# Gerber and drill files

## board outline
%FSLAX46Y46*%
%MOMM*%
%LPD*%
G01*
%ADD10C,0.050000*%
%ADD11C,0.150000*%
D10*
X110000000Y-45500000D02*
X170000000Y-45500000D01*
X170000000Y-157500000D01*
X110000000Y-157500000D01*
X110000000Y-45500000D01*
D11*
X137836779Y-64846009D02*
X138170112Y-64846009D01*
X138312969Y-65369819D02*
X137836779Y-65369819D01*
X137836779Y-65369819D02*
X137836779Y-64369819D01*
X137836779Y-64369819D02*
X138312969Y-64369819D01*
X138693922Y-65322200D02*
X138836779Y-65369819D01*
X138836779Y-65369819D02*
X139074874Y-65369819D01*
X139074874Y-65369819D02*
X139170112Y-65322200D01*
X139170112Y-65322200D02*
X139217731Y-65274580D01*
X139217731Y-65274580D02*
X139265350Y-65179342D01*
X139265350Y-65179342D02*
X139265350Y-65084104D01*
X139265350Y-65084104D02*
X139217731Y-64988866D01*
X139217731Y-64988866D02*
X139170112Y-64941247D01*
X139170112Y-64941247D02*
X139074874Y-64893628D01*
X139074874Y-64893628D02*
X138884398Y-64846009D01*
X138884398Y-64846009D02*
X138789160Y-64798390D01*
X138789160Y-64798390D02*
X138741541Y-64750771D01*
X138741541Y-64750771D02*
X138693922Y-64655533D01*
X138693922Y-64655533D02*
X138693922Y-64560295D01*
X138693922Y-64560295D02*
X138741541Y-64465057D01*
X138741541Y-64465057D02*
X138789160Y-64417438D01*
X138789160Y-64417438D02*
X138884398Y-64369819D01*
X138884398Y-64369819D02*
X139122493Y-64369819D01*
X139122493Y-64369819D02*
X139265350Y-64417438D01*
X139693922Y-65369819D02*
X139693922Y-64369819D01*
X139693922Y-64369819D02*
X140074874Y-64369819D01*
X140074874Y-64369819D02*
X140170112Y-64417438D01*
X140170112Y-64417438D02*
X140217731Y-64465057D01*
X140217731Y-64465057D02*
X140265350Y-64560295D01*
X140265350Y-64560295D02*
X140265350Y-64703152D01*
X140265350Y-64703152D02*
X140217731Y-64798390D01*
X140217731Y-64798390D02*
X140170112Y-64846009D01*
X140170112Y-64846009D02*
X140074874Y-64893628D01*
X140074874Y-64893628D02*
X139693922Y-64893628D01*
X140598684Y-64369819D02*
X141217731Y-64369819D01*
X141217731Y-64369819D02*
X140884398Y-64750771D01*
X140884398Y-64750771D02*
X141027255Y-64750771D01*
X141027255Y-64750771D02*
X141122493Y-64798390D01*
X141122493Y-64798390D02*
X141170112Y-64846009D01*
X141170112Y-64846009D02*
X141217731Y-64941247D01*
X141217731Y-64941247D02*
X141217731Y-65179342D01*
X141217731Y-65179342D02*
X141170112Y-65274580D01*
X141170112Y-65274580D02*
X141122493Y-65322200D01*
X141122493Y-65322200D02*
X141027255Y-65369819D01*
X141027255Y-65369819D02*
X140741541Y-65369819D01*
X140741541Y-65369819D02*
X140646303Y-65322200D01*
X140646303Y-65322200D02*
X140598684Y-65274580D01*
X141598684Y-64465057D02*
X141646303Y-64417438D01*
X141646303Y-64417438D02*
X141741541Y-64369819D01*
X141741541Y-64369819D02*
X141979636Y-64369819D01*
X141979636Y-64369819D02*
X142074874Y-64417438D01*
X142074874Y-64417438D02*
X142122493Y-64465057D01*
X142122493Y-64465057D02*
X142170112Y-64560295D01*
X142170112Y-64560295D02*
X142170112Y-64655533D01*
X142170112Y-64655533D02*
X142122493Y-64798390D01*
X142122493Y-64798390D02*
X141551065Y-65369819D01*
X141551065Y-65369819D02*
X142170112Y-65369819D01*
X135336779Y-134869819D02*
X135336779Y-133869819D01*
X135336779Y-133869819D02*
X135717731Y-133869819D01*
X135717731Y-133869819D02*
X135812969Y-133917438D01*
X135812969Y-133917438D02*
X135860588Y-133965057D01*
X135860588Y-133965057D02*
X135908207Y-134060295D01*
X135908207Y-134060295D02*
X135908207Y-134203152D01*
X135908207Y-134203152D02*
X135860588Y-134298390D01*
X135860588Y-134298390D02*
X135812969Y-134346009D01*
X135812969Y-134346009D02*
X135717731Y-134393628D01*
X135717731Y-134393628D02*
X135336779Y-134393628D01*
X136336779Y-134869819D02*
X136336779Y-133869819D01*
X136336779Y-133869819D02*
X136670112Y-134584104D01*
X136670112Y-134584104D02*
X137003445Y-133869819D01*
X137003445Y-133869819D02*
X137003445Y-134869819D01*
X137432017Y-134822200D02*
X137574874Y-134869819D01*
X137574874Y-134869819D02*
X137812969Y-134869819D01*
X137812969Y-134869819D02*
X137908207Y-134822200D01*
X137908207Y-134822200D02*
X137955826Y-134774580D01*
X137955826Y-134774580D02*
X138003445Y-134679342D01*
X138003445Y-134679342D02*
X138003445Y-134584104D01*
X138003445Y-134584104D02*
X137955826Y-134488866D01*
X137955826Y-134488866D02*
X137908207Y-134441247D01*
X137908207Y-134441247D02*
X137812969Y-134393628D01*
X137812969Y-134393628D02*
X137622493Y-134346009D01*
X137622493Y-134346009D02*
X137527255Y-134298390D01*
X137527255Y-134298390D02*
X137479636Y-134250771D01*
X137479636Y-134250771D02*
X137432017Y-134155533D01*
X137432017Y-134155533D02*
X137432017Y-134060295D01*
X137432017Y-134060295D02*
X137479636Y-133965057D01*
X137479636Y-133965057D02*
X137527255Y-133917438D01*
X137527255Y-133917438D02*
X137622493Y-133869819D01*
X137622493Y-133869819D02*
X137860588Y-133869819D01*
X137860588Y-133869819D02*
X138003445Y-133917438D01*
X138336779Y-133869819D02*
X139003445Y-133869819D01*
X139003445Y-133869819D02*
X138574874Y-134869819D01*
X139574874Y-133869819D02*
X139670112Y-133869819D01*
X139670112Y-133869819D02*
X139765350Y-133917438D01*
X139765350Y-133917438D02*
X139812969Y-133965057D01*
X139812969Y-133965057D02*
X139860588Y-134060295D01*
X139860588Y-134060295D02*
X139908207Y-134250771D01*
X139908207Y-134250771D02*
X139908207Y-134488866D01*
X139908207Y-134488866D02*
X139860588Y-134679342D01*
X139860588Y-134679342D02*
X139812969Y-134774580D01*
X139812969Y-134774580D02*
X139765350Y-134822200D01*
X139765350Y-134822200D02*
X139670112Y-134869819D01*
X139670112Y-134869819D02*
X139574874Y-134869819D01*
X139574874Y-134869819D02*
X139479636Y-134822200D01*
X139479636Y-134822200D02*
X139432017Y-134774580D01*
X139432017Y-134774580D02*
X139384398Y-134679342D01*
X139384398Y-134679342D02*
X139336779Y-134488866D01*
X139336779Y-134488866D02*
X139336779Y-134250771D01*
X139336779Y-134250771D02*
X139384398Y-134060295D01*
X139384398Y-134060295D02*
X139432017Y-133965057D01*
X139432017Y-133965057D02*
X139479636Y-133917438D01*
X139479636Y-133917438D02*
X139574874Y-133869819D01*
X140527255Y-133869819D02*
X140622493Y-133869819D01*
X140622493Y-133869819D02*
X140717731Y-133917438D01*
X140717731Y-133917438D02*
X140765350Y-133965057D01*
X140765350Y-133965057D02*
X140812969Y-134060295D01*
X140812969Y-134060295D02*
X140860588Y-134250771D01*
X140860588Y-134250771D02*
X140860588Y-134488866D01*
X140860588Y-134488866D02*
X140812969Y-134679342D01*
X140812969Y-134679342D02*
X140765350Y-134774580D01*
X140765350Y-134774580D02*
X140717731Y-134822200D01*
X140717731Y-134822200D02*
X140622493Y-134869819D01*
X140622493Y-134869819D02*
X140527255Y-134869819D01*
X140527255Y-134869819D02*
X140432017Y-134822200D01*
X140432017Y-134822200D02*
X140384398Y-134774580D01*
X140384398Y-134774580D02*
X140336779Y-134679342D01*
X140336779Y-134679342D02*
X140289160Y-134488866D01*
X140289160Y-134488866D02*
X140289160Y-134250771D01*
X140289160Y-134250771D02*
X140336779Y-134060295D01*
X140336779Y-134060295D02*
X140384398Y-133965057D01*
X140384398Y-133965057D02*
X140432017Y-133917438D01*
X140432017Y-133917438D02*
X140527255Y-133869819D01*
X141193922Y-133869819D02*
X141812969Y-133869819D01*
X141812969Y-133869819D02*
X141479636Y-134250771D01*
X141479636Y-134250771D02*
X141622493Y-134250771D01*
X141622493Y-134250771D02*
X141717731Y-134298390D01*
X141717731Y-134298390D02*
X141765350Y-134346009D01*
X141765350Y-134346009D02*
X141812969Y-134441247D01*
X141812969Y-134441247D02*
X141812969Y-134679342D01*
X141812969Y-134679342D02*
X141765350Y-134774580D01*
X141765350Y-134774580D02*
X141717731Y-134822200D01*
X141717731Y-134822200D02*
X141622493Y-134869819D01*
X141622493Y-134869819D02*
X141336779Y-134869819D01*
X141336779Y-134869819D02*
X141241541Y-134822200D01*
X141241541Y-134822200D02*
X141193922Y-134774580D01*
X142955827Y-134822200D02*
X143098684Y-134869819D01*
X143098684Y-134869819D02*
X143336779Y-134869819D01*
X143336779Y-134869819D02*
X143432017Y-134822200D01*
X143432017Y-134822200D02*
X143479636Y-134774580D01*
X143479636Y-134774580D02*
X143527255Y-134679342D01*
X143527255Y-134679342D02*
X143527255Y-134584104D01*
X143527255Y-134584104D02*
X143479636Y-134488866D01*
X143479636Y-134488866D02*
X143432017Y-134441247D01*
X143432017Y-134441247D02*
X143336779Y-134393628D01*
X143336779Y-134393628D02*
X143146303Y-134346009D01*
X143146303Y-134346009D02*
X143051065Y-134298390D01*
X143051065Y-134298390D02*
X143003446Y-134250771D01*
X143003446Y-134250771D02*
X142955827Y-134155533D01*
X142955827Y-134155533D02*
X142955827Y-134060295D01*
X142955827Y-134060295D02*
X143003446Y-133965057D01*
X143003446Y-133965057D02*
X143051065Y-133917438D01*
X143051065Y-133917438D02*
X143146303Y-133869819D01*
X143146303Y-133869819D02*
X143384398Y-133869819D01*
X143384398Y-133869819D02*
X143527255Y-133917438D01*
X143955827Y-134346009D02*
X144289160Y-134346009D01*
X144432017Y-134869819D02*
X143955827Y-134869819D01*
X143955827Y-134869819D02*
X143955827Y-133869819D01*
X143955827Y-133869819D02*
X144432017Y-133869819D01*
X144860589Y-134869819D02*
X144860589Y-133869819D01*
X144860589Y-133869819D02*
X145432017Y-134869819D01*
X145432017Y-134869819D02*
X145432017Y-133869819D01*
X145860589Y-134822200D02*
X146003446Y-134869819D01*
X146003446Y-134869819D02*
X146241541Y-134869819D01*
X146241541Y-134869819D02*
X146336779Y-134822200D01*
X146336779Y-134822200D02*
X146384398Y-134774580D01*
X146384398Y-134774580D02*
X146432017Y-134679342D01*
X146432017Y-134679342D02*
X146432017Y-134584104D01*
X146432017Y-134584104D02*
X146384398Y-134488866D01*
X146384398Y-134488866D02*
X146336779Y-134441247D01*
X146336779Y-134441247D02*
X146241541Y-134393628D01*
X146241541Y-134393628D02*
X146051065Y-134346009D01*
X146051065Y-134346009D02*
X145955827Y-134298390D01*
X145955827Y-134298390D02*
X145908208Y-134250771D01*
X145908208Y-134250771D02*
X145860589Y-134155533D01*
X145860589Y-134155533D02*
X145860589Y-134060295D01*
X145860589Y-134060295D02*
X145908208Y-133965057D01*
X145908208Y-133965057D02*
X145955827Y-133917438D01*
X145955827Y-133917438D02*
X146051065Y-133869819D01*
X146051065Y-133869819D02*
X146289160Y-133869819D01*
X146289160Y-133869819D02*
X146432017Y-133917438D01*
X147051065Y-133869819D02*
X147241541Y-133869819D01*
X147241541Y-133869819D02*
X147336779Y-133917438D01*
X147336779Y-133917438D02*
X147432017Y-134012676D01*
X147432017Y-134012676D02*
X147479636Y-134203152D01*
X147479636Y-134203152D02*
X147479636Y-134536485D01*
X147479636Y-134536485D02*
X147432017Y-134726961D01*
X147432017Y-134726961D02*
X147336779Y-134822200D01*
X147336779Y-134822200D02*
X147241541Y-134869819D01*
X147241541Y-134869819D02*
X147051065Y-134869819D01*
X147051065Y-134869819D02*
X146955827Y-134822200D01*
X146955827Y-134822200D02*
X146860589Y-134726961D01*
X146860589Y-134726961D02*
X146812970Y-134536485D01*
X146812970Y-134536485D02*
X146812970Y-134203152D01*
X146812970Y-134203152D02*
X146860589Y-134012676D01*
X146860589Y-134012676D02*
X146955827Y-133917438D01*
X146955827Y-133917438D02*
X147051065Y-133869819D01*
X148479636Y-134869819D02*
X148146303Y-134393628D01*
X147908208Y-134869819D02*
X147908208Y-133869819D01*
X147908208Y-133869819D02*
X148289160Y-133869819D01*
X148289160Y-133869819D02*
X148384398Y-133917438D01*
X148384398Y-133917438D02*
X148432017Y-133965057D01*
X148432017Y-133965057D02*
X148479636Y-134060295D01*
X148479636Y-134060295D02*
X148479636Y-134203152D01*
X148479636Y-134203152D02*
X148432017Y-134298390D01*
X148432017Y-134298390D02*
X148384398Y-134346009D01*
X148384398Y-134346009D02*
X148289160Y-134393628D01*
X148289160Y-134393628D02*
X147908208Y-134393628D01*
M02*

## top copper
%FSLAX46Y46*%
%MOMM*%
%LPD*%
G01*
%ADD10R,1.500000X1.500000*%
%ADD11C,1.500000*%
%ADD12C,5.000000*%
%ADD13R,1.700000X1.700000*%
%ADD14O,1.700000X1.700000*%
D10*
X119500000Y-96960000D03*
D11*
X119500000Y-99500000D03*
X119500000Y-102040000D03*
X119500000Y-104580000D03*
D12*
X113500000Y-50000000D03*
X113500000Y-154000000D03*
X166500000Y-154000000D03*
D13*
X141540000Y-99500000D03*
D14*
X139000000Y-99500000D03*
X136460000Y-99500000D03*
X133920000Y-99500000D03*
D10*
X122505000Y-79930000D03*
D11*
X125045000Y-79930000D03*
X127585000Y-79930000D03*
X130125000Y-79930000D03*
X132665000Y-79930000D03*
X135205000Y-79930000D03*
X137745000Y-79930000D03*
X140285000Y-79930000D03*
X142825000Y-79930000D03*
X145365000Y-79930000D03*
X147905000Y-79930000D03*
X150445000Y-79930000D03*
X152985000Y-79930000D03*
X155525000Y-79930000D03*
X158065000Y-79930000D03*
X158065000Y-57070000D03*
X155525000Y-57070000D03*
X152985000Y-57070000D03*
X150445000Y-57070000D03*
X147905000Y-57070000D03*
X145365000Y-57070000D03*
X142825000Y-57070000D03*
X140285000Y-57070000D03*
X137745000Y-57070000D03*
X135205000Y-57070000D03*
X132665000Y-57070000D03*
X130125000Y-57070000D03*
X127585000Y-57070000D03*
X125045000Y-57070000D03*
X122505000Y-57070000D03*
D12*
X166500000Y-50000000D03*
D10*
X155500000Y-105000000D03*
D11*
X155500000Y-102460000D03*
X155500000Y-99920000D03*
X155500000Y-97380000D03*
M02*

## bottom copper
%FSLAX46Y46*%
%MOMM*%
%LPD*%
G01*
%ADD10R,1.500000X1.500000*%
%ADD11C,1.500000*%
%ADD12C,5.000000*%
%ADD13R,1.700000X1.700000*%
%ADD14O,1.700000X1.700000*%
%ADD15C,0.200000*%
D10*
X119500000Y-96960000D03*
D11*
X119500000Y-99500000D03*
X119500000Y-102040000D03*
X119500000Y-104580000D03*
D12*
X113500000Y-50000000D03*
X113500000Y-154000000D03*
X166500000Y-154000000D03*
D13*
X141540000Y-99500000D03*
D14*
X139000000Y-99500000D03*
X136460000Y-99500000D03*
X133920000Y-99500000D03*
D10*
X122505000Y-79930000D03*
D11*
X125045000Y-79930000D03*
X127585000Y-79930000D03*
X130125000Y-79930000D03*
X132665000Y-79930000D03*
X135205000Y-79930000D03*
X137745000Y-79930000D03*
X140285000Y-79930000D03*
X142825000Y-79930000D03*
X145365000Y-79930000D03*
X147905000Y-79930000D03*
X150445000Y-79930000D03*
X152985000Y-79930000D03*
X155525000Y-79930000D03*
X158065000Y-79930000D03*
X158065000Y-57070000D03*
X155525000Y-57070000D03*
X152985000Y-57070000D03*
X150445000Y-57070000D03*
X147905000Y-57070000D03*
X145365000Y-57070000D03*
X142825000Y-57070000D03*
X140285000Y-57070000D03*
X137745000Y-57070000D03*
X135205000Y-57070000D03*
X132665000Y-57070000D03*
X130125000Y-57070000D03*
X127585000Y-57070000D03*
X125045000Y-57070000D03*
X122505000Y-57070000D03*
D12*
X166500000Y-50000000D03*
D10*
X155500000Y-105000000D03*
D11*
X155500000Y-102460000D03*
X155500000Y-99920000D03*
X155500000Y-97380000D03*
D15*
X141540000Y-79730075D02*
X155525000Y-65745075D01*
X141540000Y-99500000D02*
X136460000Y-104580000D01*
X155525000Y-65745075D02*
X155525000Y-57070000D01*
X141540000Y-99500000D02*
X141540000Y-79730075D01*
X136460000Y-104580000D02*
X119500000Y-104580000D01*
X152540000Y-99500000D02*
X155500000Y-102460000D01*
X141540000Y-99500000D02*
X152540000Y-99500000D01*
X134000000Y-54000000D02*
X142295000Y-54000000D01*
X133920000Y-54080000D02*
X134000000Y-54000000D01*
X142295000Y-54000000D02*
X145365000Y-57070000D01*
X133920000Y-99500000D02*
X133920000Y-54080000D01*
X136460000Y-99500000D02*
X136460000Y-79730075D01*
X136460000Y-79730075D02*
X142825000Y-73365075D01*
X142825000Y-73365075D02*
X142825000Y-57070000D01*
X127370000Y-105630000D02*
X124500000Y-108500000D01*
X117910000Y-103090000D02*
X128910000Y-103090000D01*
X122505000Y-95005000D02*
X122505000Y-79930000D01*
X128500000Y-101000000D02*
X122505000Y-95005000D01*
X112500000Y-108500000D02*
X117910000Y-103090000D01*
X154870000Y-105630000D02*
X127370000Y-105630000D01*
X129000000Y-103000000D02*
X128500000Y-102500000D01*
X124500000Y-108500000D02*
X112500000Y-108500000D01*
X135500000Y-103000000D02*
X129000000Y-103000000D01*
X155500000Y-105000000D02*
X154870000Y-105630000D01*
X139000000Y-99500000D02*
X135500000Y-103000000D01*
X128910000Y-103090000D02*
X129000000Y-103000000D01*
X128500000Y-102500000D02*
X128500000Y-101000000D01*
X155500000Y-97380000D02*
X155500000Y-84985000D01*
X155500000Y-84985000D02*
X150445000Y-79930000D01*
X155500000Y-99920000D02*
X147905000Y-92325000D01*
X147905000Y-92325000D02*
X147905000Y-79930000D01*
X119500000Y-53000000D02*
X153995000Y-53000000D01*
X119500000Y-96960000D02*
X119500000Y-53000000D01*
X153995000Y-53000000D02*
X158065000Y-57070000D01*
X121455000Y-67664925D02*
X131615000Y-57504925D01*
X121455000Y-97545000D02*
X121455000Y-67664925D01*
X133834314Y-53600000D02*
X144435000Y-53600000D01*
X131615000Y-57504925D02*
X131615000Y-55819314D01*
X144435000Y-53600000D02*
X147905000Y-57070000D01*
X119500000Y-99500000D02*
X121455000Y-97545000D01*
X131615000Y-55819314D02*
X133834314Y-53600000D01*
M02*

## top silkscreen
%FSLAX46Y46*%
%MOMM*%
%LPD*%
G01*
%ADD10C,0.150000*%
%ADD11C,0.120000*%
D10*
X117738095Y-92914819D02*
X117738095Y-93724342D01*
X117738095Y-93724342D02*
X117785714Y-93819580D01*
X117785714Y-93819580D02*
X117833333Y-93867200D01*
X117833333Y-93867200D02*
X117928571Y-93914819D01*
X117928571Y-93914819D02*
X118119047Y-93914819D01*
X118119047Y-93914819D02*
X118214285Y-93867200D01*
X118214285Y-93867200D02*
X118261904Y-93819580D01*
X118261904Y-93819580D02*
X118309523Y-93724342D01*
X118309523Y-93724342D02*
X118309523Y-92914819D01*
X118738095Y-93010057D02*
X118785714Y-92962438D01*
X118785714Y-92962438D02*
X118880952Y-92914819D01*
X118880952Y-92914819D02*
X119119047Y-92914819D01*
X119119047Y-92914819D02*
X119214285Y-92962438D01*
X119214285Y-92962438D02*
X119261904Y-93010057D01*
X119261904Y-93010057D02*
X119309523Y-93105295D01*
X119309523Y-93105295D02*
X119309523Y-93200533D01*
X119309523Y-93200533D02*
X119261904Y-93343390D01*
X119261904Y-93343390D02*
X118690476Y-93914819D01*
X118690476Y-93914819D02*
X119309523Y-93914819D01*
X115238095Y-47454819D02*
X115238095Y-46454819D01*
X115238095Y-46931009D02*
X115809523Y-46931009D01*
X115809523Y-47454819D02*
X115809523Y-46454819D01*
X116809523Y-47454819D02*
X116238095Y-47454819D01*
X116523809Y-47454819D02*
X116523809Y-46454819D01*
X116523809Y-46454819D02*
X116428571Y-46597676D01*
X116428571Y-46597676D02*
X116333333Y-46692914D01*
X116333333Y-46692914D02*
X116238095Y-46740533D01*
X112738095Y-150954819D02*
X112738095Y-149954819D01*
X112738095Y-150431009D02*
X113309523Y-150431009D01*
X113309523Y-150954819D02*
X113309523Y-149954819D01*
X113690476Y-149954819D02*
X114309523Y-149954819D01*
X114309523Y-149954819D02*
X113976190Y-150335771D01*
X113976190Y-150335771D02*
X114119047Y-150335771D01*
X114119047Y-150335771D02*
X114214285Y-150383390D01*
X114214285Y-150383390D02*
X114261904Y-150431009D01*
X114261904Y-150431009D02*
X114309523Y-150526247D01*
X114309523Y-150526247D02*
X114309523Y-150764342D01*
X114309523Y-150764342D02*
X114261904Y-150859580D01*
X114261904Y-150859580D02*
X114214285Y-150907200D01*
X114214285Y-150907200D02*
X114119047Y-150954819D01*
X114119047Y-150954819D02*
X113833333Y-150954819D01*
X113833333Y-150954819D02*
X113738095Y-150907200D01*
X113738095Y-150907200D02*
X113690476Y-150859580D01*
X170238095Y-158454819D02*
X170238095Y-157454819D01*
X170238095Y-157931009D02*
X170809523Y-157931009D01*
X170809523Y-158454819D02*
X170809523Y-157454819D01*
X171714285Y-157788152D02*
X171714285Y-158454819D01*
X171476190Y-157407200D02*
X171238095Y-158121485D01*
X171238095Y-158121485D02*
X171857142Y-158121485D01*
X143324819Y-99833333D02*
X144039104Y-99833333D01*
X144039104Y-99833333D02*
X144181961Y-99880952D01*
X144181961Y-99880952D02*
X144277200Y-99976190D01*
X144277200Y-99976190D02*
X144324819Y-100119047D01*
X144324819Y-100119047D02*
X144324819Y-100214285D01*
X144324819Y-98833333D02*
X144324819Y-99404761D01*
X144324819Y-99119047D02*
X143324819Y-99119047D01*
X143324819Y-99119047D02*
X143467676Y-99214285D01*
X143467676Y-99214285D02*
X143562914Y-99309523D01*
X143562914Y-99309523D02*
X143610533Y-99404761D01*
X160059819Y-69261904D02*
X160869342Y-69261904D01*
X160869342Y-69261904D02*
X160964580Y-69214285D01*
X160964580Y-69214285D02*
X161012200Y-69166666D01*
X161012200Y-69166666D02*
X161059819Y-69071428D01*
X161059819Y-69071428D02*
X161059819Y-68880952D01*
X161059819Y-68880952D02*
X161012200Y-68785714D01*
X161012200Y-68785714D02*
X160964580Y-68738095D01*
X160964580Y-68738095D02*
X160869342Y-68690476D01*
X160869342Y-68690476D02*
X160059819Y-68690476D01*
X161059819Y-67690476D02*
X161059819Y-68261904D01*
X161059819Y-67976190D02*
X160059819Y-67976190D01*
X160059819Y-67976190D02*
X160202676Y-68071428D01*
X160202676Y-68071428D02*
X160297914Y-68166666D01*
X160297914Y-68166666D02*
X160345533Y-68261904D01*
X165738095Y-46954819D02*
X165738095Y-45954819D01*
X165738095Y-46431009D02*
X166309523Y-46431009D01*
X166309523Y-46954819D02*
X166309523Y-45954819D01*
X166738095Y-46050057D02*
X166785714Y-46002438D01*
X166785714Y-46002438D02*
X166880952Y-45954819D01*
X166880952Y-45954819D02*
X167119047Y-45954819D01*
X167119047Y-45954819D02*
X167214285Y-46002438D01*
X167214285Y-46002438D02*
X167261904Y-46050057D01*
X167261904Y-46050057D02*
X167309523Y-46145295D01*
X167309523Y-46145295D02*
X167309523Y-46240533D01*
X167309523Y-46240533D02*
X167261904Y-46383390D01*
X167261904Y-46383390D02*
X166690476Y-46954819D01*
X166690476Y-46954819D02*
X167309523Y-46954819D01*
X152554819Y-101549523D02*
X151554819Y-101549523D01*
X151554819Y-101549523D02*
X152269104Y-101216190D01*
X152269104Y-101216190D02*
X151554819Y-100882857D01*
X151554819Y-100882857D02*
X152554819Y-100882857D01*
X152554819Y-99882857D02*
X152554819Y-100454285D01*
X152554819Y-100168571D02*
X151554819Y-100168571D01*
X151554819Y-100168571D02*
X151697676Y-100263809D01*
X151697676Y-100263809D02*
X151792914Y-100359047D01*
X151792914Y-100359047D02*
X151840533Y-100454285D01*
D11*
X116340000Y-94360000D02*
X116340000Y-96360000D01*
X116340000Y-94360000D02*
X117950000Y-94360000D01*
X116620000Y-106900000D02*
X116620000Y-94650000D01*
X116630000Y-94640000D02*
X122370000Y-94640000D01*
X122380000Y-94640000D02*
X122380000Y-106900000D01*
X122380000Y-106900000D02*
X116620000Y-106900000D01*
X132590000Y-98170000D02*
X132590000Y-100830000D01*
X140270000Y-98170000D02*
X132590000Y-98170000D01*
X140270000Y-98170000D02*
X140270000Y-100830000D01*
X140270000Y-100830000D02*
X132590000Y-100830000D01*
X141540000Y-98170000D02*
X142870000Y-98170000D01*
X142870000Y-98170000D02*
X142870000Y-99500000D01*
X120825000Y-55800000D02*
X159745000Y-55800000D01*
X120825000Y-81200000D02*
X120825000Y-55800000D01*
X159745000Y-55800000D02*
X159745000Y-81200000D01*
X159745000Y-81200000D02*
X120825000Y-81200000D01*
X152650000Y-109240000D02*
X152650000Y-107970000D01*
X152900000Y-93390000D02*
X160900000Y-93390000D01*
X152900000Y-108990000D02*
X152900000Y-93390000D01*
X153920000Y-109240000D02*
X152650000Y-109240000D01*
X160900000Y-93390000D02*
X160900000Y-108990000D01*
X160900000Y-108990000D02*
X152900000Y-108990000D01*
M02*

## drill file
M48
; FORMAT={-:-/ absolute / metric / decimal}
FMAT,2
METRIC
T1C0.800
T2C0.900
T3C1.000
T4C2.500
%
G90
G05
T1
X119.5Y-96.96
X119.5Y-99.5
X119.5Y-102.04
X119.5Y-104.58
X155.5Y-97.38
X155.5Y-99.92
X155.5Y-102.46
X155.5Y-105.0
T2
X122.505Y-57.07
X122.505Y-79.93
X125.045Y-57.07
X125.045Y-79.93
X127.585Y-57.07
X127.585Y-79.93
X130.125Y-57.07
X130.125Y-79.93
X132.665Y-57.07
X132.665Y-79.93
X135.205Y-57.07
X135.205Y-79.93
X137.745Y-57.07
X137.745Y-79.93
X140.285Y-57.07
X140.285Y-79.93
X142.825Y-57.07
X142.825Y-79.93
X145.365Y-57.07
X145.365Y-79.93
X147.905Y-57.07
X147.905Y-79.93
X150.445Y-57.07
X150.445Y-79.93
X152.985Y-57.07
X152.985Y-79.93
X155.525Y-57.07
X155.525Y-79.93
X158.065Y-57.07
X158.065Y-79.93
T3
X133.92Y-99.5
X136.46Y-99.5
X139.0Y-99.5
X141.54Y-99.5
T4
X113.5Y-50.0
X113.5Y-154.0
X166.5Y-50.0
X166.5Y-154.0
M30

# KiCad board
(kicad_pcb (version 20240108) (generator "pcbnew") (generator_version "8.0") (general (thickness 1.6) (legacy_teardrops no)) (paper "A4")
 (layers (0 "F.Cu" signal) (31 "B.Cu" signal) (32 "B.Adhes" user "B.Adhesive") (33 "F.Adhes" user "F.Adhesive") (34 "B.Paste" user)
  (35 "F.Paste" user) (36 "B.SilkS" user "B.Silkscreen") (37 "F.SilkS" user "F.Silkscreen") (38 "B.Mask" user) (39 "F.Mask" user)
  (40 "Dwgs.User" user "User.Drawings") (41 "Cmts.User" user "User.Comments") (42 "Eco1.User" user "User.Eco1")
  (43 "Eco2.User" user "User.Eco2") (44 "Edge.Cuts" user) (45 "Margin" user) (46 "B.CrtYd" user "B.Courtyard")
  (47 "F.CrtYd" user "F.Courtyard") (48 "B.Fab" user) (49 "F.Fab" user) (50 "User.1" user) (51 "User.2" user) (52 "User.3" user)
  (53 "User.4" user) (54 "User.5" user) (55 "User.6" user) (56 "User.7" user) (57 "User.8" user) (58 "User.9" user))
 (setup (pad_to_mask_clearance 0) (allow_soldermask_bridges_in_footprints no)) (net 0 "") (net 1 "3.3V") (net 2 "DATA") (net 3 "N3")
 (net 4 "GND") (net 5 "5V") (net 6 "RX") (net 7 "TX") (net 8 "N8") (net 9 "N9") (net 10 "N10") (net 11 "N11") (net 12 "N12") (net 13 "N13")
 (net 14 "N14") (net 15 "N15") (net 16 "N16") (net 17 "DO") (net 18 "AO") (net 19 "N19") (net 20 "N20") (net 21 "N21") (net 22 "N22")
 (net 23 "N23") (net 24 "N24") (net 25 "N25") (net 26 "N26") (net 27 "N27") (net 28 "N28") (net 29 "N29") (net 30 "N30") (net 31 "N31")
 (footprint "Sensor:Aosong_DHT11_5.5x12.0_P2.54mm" (layer "F.Cu") (at 119.5 96.96)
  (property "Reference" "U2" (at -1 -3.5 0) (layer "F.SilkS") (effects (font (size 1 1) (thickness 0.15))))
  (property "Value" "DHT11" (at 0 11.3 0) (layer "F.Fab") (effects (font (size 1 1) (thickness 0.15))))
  (fp_line (start -3.16 -2.6) (end -3.16 -0.6) (stroke (width 0.12) (type solid)) (layer "F.SilkS"))
  (fp_line (start -3.16 -2.6) (end -1.55 -2.6) (stroke (width 0.12) (type solid)) (layer "F.SilkS"))
  (fp_line (start -2.88 9.94) (end -2.88 -2.31) (stroke (width 0.12) (type solid)) (layer "F.SilkS"))
  (fp_line (start -2.87 -2.32) (end 2.87 -2.32) (stroke (width 0.12) (type solid)) (layer "F.SilkS"))
  (fp_line (start 2.88 -2.32) (end 2.88 9.94) (stroke (width 0.12) (type solid)) (layer "F.SilkS"))
  (fp_line (start 2.88 9.94) (end -2.88 9.94) (stroke (width 0.12) (type solid)) (layer "F.SilkS"))
  (pad "1" thru_hole rect (at 0 0) (size 1.5 1.5) (drill 0.8) (layers "*.Cu" "*.Mask") (remove_unused_layers no) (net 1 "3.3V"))
  (pad "2" thru_hole circle (at 0 2.54) (size 1.5 1.5) (drill 0.8) (layers "*.Cu" "*.Mask") (remove_unused_layers no) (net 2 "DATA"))
  (pad "3" thru_hole circle (at 0 5.08) (size 1.5 1.5) (drill 0.8) (layers "*.Cu" "*.Mask") (remove_unused_layers no) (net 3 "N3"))
  (pad "4" thru_hole circle (at 0 7.62) (size 1.5 1.5) (drill 0.8) (layers "*.Cu" "*.Mask") (remove_unused_layers no) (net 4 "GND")))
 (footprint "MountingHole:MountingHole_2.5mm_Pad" (layer "F.Cu") (at 113.5 50)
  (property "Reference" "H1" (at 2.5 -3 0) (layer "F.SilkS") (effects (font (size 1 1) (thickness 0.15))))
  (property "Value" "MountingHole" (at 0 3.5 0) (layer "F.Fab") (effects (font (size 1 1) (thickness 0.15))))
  (pad "1" thru_hole circle (at 0 0) (size 5 5) (drill 2.5) (layers "*.Cu" "*.Mask") (remove_unused_layers no)))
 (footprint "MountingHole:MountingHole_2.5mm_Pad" (layer "F.Cu") (at 113.5 154)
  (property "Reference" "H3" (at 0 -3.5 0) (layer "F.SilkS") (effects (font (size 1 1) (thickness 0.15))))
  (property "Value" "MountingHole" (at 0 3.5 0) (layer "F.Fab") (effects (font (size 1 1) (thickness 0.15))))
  (pad "1" thru_hole circle (at 0 0) (size 5 5) (drill 2.5) (layers "*.Cu" "*.Mask") (remove_unused_layers no)))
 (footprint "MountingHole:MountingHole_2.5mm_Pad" (layer "F.Cu") (at 166.5 154)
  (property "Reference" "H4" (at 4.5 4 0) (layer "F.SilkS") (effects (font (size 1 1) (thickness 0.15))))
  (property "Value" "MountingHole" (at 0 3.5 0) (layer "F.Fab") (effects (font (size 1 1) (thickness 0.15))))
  (pad "1" thru_hole circle (at 0 0) (size 5 5) (drill 2.5) (layers "*.Cu" "*.Mask") (remove_unused_layers no)))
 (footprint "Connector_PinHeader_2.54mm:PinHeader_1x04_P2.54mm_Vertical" (layer "F.Cu") (at 141.54 99.5 -90)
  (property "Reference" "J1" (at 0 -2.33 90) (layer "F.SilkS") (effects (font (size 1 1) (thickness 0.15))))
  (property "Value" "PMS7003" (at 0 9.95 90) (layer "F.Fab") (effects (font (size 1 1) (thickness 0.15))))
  (fp_line (start -1.33 8.95) (end 1.33 8.95) (stroke (width 0.12) (type solid)) (layer "F.SilkS"))
  (fp_line (start -1.33 1.27) (end -1.33 8.95) (stroke (width 0.12) (type solid)) (layer "F.SilkS"))
  (fp_line (start -1.33 1.27) (end 1.33 1.27) (stroke (width 0.12) (type solid)) (layer "F.SilkS"))
  (fp_line (start 1.33 1.27) (end 1.33 8.95) (stroke (width 0.12) (type solid)) (layer "F.SilkS"))
  (fp_line (start -1.33 0) (end -1.33 -1.33) (stroke (width 0.12) (type solid)) (layer "F.SilkS"))
  (fp_line (start -1.33 -1.33) (end 0 -1.33) (stroke (width 0.12) (type solid)) (layer "F.SilkS"))
  (pad "1" thru_hole rect (at 0 0 270) (size 1.7 1.7) (drill 1) (layers "*.Cu" "*.Mask") (remove_unused_layers no) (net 4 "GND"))
  (pad "2" thru_hole oval (at 0 2.54 270) (size 1.7 1.7) (drill 1) (layers "*.Cu" "*.Mask") (remove_unused_layers no) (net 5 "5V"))
  (pad "3" thru_hole oval (at 0 5.08 270) (size 1.7 1.7) (drill 1) (layers "*.Cu" "*.Mask") (remove_unused_layers no) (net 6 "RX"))
  (pad "4" thru_hole oval (at 0 7.62 270) (size 1.7 1.7) (drill 1) (layers "*.Cu" "*.Mask") (remove_unused_layers no) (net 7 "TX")))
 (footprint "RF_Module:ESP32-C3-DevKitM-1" (layer "F.Cu") (at 122.505 79.93 90)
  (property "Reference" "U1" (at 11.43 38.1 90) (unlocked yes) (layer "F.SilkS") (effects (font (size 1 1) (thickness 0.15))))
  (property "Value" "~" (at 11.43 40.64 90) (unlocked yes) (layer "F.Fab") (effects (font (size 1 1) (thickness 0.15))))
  (fp_line (start 24.13 -1.68) (end 24.13 37.24) (stroke (width 0.12) (type solid)) (layer "F.SilkS"))
  (fp_line (start -1.27 -1.68) (end 24.13 -1.68) (stroke (width 0.12) (type solid)) (layer "F.SilkS"))
  (fp_line (start 24.13 37.24) (end -1.27 37.24) (stroke (width 0.12) (type solid)) (layer "F.SilkS"))
  (fp_line (start -1.27 37.24) (end -1.27 -1.68) (stroke (width 0.12) (type solid)) (layer "F.SilkS"))
  (pad "1" thru_hole rect (at 0 0 90) (size 1.5 1.5) (drill 0.9) (layers "*.Cu" "*.Mask") (remove_unused_layers yes) (keep_end_layers yes)
   (zone_layer_connections) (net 5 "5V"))
  (pad "2" thru_hole circle (at 0 2.54 90) (size 1.5 1.5) (drill 0.9) (layers "*.Cu" "*.Mask") (remove_unused_layers yes)
   (keep_end_layers yes) (zone_layer_connections) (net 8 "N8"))
  (pad "3" thru_hole circle (at 0 5.08 90) (size 1.5 1.5) (drill 0.9) (layers "*.Cu" "*.Mask") (remove_unused_layers yes)
   (keep_end_layers yes) (zone_layer_connections) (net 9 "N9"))
  (pad "4" thru_hole circle (at 0 7.62 90) (size 1.5 1.5) (drill 0.9) (layers "*.Cu" "*.Mask") (remove_unused_layers yes)
   (keep_end_layers yes) (zone_layer_connections) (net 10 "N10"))
  (pad "5" thru_hole circle (at 0 10.16 90) (size 1.5 1.5) (drill 0.9) (layers "*.Cu" "*.Mask") (remove_unused_layers yes)
   (keep_end_layers yes) (zone_layer_connections) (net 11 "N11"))
  (pad "6" thru_hole circle (at 0 12.7 90) (size 1.5 1.5) (drill 0.9) (layers "*.Cu" "*.Mask") (remove_unused_layers yes)
   (keep_end_layers yes) (zone_layer_connections) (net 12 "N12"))
  (pad "7" thru_hole circle (at 0 15.24 90) (size 1.5 1.5) (drill 0.9) (layers "*.Cu" "*.Mask") (remove_unused_layers yes)
   (keep_end_layers yes) (zone_layer_connections) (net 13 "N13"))
  (pad "8" thru_hole circle (at 0 17.78 90) (size 1.5 1.5) (drill 0.9) (layers "*.Cu" "*.Mask") (remove_unused_layers yes)
   (keep_end_layers yes) (zone_layer_connections) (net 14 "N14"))
  (pad "9" thru_hole circle (at 0 20.32 90) (size 1.5 1.5) (drill 0.9) (layers "*.Cu" "*.Mask") (remove_unused_layers yes)
   (keep_end_layers yes) (zone_layer_connections) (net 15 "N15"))
  (pad "10" thru_hole circle (at 0 22.86 90) (size 1.5 1.5) (drill 0.9) (layers "*.Cu" "*.Mask") (remove_unused_layers yes)
   (keep_end_layers yes) (zone_layer_connections) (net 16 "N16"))
  (pad "11" thru_hole circle (at 0 25.4 90) (size 1.5 1.5) (drill 0.9) (layers "*.Cu" "*.Mask") (remove_unused_layers yes)
   (keep_end_layers yes) (zone_layer_connections) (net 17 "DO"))
  (pad "12" thru_hole circle (at 0 27.94 90) (size 1.5 1.5) (drill 0.9) (layers "*.Cu" "*.Mask") (remove_unused_layers yes)
   (keep_end_layers yes) (zone_layer_connections) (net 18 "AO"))
  (pad "13" thru_hole circle (at 0 30.48 90) (size 1.5 1.5) (drill 0.9) (layers "*.Cu" "*.Mask") (remove_unused_layers yes)
   (keep_end_layers yes) (zone_layer_connections) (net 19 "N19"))
  (pad "14" thru_hole circle (at 0 33.02 90) (size 1.5 1.5) (drill 0.9) (layers "*.Cu" "*.Mask") (remove_unused_layers yes)
   (keep_end_layers yes) (zone_layer_connections) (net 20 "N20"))
  (pad "15" thru_hole circle (at 0 35.56 90) (size 1.5 1.5) (drill 0.9) (layers "*.Cu" "*.Mask") (remove_unused_layers yes)
   (keep_end_layers yes) (zone_layer_connections) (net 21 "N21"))
  (pad "16" thru_hole circle (at 22.86 35.56 90) (size 1.5 1.5) (drill 0.9) (layers "*.Cu" "*.Mask") (remove_unused_layers yes)
   (keep_end_layers yes) (zone_layer_connections) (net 1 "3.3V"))
  (pad "17" thru_hole circle (at 22.86 33.02 90) (size 1.5 1.5) (drill 0.9) (layers "*.Cu" "*.Mask") (remove_unused_layers yes)
   (keep_end_layers yes) (zone_layer_connections) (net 4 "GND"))
  (pad "18" thru_hole circle (at 22.86 30.48 90) (size 1.5 1.5) (drill 0.9) (layers "*.Cu" "*.Mask") (remove_unused_layers yes)
   (keep_end_layers yes) (zone_layer_connections) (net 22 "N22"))
  (pad "19" thru_hole circle (at 22.86 27.94 90) (size 1.5 1.5) (drill 0.9) (layers "*.Cu" "*.Mask") (remove_unused_layers yes)
   (keep_end_layers yes) (zone_layer_connections) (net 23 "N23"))
  (pad "20" thru_hole circle (at 22.86 25.4 90) (size 1.5 1.5) (drill 0.9) (layers "*.Cu" "*.Mask") (remove_unused_layers yes)
   (keep_end_layers yes) (zone_layer_connections) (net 2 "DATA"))
  (pad "21" thru_hole circle (at 22.86 22.86 90) (size 1.5 1.5) (drill 0.9) (layers "*.Cu" "*.Mask") (remove_unused_layers yes)
   (keep_end_layers yes) (zone_layer_connections) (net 7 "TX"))
  (pad "22" thru_hole circle (at 22.86 20.32 90) (size 1.5 1.5) (drill 0.9) (layers "*.Cu" "*.Mask") (remove_unused_layers yes)
   (keep_end_layers yes) (zone_layer_connections) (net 6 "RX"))
  (pad "23" thru_hole circle (at 22.86 17.78 90) (size 1.5 1.5) (drill 0.9) (layers "*.Cu" "*.Mask") (remove_unused_layers yes)
   (keep_end_layers yes) (zone_layer_connections) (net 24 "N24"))
  (pad "24" thru_hole circle (at 22.86 15.24 90) (size 1.5 1.5) (drill 0.9) (layers "*.Cu" "*.Mask") (remove_unused_layers yes)
   (keep_end_layers yes) (zone_layer_connections) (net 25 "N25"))
  (pad "25" thru_hole circle (at 22.86 12.7 90) (size 1.5 1.5) (drill 0.9) (layers "*.Cu" "*.Mask") (remove_unused_layers yes)
   (keep_end_layers yes) (zone_layer_connections) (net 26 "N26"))
  (pad "26" thru_hole circle (at 22.86 10.16 90) (size 1.5 1.5) (drill 0.9) (layers "*.Cu" "*.Mask") (remove_unused_layers yes)
   (keep_end_layers yes) (zone_layer_connections) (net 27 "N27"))
  (pad "27" thru_hole circle (at 22.86 7.62 90) (size 1.5 1.5) (drill 0.9) (layers "*.Cu" "*.Mask") (remove_unused_layers yes)
   (keep_end_layers yes) (zone_layer_connections) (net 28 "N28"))
  (pad "28" thru_hole circle (at 22.86 5.08 90) (size 1.5 1.5) (drill 0.9) (layers "*.Cu" "*.Mask") (remove_unused_layers yes)
   (keep_end_layers yes) (zone_layer_connections) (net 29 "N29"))
  (pad "29" thru_hole circle (at 22.86 2.54 90) (size 1.5 1.5) (drill 0.9) (layers "*.Cu" "*.Mask") (remove_unused_layers yes)
   (keep_end_layers yes) (zone_layer_connections) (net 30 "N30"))
  (pad "30" thru_hole circle (at 22.86 0 90) (size 1.5 1.5) (drill 0.9) (layers "*.Cu" "*.Mask") (remove_unused_layers yes)
   (keep_end_layers yes) (zone_layer_connections) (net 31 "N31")))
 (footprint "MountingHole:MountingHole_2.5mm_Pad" (layer "F.Cu") (at 166.5 50)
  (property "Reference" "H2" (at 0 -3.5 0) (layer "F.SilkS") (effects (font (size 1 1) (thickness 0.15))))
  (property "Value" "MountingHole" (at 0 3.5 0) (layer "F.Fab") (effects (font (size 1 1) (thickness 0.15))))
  (pad "1" thru_hole circle (at 0 0) (size 5 5) (drill 2.5) (layers "*.Cu" "*.Mask") (remove_unused_layers no)))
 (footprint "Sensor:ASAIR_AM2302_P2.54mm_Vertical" (layer "F.Cu") (at 155.5 105 90)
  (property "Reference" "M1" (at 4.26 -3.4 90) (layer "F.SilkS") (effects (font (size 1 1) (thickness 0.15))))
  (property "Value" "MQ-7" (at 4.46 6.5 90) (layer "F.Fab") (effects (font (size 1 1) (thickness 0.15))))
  (fp_line (start -4.24 -2.85) (end -2.97 -2.85) (stroke (width 0.12) (type solid)) (layer "F.SilkS"))
  (fp_line (start 11.61 -2.6) (end 11.61 5.4) (stroke (width 0.12) (type solid)) (layer "F.SilkS"))
  (fp_line (start -3.99 -2.6) (end 11.61 -2.6) (stroke (width 0.12) (type solid)) (layer "F.SilkS"))
  (fp_line (start -4.24 -1.58) (end -4.24 -2.85) (stroke (width 0.12) (type solid)) (layer "F.SilkS"))
  (fp_line (start 11.61 5.4) (end -3.99 5.4) (stroke (width 0.12) (type solid)) (layer "F.SilkS"))
  (fp_line (start -3.99 5.4) (end -3.99 -2.6) (stroke (width 0.12) (type solid)) (layer "F.SilkS"))
  (pad "1" thru_hole rect (at 0 0 180) (size 1.5 1.5) (drill 0.8) (layers "*.Cu" "*.Mask") (remove_unused_layers no) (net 5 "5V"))
  (pad "2" thru_hole circle (at 2.54 0 180) (size 1.5 1.5) (drill 0.8) (layers "*.Cu" "*.Mask") (remove_unused_layers no) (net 4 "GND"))
  (pad "3" thru_hole circle (at 5.08 0 180) (size 1.5 1.5) (drill 0.8) (layers "*.Cu" "*.Mask") (remove_unused_layers no) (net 17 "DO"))
  (pad "4" thru_hole circle (at 7.62 0 180) (size 1.5 1.5) (drill 0.8) (layers "*.Cu" "*.Mask") (remove_unused_layers no) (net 18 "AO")))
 (gr_rect (start 110 45.5) (end 170 157.5) (stroke (width 0.05) (type default)) (fill none) (layer "Edge.Cuts"))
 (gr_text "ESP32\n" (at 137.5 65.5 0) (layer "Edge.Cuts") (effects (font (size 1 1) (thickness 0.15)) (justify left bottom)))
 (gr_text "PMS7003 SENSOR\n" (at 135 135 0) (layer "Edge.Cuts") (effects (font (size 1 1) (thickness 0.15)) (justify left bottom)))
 (segment (start 141.54 79.730075) (end 155.525 65.745075) (width 0.2) (layer "B.Cu") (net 4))
 (segment (start 141.54 99.5) (end 136.46 104.58) (width 0.2) (layer "B.Cu") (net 4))
 (segment (start 155.525 65.745075) (end 155.525 57.07) (width 0.2) (layer "B.Cu") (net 4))
 (segment (start 141.54 99.5) (end 141.54 79.730075) (width 0.2) (layer "B.Cu") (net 4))
 (segment (start 136.46 104.58) (end 119.5 104.58) (width 0.2) (layer "B.Cu") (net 4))
 (segment (start 152.54 99.5) (end 155.5 102.46) (width 0.2) (layer "B.Cu") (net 4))
 (segment (start 141.54 99.5) (end 152.54 99.5) (width 0.2) (layer "B.Cu") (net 4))
 (segment (start 134 54) (end 142.295 54) (width 0.2) (layer "B.Cu") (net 7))
 (segment (start 133.92 54.08) (end 134 54) (width 0.2) (layer "B.Cu") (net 7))
 (segment (start 142.295 54) (end 145.365 57.07) (width 0.2) (layer "B.Cu") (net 7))
 (segment (start 133.92 99.5) (end 133.92 54.08) (width 0.2) (layer "B.Cu") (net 7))
 (segment (start 136.46 99.5) (end 136.46 79.730075) (width 0.2) (layer "B.Cu") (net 6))
 (segment (start 136.46 79.730075) (end 142.825 73.365075) (width 0.2) (layer "B.Cu") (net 6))
 (segment (start 142.825 73.365075) (end 142.825 57.07) (width 0.2) (layer "B.Cu") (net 6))
 (segment (start 127.37 105.63) (end 124.5 108.5) (width 0.2) (layer "B.Cu") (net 5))
 (segment (start 117.91 103.09) (end 128.91 103.09) (width 0.2) (layer "B.Cu") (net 5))
 (segment (start 122.505 95.005) (end 122.505 79.93) (width 0.2) (layer "B.Cu") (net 5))
 (segment (start 128.5 101) (end 122.505 95.005) (width 0.2) (layer "B.Cu") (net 5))
 (segment (start 112.5 108.5) (end 117.91 103.09) (width 0.2) (layer "B.Cu") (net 5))
 (segment (start 154.87 105.63) (end 127.37 105.63) (width 0.2) (layer "B.Cu") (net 5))
 (segment (start 129 103) (end 128.5 102.5) (width 0.2) (layer "B.Cu") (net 5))
 (segment (start 124.5 108.5) (end 112.5 108.5) (width 0.2) (layer "B.Cu") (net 5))
 (segment (start 135.5 103) (end 129 103) (width 0.2) (layer "B.Cu") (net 5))
 (segment (start 155.5 105) (end 154.87 105.63) (width 0.2) (layer "B.Cu") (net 5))
 (segment (start 139 99.5) (end 135.5 103) (width 0.2) (layer "B.Cu") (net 5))
 (segment (start 128.91 103.09) (end 129 103) (width 0.2) (layer "B.Cu") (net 5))
 (segment (start 128.5 102.5) (end 128.5 101) (width 0.2) (layer "B.Cu") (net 5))
 (segment (start 155.5 97.38) (end 155.5 84.985) (width 0.2) (layer "B.Cu") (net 18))
 (segment (start 155.5 84.985) (end 150.445 79.93) (width 0.2) (layer "B.Cu") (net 18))
 (segment (start 155.5 99.92) (end 147.905 92.325) (width 0.2) (layer "B.Cu") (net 17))
 (segment (start 147.905 92.325) (end 147.905 79.93) (width 0.2) (layer "B.Cu") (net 17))
 (segment (start 119.5 53) (end 153.995 53) (width 0.2) (layer "B.Cu") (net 1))
 (segment (start 119.5 96.96) (end 119.5 53) (width 0.2) (layer "B.Cu") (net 1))
 (segment (start 153.995 53) (end 158.065 57.07) (width 0.2) (layer "B.Cu") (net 1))
 (segment (start 121.455 67.664925) (end 131.615 57.504925) (width 0.2) (layer "B.Cu") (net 2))
 (segment (start 121.455 97.545) (end 121.455 67.664925) (width 0.2) (layer "B.Cu") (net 2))
 (segment (start 133.834314 53.6) (end 144.435 53.6) (width 0.2) (layer "B.Cu") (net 2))
 (segment (start 131.615 57.504925) (end 131.615 55.819314) (width 0.2) (layer "B.Cu") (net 2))
 (segment (start 144.435 53.6) (end 147.905 57.07) (width 0.2) (layer "B.Cu") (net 2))
 (segment (start 119.5 99.5) (end 121.455 97.545) (width 0.2) (layer "B.Cu") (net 2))
 (segment (start 131.615 55.819314) (end 133.834314 53.6) (width 0.2) (layer "B.Cu") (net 2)))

